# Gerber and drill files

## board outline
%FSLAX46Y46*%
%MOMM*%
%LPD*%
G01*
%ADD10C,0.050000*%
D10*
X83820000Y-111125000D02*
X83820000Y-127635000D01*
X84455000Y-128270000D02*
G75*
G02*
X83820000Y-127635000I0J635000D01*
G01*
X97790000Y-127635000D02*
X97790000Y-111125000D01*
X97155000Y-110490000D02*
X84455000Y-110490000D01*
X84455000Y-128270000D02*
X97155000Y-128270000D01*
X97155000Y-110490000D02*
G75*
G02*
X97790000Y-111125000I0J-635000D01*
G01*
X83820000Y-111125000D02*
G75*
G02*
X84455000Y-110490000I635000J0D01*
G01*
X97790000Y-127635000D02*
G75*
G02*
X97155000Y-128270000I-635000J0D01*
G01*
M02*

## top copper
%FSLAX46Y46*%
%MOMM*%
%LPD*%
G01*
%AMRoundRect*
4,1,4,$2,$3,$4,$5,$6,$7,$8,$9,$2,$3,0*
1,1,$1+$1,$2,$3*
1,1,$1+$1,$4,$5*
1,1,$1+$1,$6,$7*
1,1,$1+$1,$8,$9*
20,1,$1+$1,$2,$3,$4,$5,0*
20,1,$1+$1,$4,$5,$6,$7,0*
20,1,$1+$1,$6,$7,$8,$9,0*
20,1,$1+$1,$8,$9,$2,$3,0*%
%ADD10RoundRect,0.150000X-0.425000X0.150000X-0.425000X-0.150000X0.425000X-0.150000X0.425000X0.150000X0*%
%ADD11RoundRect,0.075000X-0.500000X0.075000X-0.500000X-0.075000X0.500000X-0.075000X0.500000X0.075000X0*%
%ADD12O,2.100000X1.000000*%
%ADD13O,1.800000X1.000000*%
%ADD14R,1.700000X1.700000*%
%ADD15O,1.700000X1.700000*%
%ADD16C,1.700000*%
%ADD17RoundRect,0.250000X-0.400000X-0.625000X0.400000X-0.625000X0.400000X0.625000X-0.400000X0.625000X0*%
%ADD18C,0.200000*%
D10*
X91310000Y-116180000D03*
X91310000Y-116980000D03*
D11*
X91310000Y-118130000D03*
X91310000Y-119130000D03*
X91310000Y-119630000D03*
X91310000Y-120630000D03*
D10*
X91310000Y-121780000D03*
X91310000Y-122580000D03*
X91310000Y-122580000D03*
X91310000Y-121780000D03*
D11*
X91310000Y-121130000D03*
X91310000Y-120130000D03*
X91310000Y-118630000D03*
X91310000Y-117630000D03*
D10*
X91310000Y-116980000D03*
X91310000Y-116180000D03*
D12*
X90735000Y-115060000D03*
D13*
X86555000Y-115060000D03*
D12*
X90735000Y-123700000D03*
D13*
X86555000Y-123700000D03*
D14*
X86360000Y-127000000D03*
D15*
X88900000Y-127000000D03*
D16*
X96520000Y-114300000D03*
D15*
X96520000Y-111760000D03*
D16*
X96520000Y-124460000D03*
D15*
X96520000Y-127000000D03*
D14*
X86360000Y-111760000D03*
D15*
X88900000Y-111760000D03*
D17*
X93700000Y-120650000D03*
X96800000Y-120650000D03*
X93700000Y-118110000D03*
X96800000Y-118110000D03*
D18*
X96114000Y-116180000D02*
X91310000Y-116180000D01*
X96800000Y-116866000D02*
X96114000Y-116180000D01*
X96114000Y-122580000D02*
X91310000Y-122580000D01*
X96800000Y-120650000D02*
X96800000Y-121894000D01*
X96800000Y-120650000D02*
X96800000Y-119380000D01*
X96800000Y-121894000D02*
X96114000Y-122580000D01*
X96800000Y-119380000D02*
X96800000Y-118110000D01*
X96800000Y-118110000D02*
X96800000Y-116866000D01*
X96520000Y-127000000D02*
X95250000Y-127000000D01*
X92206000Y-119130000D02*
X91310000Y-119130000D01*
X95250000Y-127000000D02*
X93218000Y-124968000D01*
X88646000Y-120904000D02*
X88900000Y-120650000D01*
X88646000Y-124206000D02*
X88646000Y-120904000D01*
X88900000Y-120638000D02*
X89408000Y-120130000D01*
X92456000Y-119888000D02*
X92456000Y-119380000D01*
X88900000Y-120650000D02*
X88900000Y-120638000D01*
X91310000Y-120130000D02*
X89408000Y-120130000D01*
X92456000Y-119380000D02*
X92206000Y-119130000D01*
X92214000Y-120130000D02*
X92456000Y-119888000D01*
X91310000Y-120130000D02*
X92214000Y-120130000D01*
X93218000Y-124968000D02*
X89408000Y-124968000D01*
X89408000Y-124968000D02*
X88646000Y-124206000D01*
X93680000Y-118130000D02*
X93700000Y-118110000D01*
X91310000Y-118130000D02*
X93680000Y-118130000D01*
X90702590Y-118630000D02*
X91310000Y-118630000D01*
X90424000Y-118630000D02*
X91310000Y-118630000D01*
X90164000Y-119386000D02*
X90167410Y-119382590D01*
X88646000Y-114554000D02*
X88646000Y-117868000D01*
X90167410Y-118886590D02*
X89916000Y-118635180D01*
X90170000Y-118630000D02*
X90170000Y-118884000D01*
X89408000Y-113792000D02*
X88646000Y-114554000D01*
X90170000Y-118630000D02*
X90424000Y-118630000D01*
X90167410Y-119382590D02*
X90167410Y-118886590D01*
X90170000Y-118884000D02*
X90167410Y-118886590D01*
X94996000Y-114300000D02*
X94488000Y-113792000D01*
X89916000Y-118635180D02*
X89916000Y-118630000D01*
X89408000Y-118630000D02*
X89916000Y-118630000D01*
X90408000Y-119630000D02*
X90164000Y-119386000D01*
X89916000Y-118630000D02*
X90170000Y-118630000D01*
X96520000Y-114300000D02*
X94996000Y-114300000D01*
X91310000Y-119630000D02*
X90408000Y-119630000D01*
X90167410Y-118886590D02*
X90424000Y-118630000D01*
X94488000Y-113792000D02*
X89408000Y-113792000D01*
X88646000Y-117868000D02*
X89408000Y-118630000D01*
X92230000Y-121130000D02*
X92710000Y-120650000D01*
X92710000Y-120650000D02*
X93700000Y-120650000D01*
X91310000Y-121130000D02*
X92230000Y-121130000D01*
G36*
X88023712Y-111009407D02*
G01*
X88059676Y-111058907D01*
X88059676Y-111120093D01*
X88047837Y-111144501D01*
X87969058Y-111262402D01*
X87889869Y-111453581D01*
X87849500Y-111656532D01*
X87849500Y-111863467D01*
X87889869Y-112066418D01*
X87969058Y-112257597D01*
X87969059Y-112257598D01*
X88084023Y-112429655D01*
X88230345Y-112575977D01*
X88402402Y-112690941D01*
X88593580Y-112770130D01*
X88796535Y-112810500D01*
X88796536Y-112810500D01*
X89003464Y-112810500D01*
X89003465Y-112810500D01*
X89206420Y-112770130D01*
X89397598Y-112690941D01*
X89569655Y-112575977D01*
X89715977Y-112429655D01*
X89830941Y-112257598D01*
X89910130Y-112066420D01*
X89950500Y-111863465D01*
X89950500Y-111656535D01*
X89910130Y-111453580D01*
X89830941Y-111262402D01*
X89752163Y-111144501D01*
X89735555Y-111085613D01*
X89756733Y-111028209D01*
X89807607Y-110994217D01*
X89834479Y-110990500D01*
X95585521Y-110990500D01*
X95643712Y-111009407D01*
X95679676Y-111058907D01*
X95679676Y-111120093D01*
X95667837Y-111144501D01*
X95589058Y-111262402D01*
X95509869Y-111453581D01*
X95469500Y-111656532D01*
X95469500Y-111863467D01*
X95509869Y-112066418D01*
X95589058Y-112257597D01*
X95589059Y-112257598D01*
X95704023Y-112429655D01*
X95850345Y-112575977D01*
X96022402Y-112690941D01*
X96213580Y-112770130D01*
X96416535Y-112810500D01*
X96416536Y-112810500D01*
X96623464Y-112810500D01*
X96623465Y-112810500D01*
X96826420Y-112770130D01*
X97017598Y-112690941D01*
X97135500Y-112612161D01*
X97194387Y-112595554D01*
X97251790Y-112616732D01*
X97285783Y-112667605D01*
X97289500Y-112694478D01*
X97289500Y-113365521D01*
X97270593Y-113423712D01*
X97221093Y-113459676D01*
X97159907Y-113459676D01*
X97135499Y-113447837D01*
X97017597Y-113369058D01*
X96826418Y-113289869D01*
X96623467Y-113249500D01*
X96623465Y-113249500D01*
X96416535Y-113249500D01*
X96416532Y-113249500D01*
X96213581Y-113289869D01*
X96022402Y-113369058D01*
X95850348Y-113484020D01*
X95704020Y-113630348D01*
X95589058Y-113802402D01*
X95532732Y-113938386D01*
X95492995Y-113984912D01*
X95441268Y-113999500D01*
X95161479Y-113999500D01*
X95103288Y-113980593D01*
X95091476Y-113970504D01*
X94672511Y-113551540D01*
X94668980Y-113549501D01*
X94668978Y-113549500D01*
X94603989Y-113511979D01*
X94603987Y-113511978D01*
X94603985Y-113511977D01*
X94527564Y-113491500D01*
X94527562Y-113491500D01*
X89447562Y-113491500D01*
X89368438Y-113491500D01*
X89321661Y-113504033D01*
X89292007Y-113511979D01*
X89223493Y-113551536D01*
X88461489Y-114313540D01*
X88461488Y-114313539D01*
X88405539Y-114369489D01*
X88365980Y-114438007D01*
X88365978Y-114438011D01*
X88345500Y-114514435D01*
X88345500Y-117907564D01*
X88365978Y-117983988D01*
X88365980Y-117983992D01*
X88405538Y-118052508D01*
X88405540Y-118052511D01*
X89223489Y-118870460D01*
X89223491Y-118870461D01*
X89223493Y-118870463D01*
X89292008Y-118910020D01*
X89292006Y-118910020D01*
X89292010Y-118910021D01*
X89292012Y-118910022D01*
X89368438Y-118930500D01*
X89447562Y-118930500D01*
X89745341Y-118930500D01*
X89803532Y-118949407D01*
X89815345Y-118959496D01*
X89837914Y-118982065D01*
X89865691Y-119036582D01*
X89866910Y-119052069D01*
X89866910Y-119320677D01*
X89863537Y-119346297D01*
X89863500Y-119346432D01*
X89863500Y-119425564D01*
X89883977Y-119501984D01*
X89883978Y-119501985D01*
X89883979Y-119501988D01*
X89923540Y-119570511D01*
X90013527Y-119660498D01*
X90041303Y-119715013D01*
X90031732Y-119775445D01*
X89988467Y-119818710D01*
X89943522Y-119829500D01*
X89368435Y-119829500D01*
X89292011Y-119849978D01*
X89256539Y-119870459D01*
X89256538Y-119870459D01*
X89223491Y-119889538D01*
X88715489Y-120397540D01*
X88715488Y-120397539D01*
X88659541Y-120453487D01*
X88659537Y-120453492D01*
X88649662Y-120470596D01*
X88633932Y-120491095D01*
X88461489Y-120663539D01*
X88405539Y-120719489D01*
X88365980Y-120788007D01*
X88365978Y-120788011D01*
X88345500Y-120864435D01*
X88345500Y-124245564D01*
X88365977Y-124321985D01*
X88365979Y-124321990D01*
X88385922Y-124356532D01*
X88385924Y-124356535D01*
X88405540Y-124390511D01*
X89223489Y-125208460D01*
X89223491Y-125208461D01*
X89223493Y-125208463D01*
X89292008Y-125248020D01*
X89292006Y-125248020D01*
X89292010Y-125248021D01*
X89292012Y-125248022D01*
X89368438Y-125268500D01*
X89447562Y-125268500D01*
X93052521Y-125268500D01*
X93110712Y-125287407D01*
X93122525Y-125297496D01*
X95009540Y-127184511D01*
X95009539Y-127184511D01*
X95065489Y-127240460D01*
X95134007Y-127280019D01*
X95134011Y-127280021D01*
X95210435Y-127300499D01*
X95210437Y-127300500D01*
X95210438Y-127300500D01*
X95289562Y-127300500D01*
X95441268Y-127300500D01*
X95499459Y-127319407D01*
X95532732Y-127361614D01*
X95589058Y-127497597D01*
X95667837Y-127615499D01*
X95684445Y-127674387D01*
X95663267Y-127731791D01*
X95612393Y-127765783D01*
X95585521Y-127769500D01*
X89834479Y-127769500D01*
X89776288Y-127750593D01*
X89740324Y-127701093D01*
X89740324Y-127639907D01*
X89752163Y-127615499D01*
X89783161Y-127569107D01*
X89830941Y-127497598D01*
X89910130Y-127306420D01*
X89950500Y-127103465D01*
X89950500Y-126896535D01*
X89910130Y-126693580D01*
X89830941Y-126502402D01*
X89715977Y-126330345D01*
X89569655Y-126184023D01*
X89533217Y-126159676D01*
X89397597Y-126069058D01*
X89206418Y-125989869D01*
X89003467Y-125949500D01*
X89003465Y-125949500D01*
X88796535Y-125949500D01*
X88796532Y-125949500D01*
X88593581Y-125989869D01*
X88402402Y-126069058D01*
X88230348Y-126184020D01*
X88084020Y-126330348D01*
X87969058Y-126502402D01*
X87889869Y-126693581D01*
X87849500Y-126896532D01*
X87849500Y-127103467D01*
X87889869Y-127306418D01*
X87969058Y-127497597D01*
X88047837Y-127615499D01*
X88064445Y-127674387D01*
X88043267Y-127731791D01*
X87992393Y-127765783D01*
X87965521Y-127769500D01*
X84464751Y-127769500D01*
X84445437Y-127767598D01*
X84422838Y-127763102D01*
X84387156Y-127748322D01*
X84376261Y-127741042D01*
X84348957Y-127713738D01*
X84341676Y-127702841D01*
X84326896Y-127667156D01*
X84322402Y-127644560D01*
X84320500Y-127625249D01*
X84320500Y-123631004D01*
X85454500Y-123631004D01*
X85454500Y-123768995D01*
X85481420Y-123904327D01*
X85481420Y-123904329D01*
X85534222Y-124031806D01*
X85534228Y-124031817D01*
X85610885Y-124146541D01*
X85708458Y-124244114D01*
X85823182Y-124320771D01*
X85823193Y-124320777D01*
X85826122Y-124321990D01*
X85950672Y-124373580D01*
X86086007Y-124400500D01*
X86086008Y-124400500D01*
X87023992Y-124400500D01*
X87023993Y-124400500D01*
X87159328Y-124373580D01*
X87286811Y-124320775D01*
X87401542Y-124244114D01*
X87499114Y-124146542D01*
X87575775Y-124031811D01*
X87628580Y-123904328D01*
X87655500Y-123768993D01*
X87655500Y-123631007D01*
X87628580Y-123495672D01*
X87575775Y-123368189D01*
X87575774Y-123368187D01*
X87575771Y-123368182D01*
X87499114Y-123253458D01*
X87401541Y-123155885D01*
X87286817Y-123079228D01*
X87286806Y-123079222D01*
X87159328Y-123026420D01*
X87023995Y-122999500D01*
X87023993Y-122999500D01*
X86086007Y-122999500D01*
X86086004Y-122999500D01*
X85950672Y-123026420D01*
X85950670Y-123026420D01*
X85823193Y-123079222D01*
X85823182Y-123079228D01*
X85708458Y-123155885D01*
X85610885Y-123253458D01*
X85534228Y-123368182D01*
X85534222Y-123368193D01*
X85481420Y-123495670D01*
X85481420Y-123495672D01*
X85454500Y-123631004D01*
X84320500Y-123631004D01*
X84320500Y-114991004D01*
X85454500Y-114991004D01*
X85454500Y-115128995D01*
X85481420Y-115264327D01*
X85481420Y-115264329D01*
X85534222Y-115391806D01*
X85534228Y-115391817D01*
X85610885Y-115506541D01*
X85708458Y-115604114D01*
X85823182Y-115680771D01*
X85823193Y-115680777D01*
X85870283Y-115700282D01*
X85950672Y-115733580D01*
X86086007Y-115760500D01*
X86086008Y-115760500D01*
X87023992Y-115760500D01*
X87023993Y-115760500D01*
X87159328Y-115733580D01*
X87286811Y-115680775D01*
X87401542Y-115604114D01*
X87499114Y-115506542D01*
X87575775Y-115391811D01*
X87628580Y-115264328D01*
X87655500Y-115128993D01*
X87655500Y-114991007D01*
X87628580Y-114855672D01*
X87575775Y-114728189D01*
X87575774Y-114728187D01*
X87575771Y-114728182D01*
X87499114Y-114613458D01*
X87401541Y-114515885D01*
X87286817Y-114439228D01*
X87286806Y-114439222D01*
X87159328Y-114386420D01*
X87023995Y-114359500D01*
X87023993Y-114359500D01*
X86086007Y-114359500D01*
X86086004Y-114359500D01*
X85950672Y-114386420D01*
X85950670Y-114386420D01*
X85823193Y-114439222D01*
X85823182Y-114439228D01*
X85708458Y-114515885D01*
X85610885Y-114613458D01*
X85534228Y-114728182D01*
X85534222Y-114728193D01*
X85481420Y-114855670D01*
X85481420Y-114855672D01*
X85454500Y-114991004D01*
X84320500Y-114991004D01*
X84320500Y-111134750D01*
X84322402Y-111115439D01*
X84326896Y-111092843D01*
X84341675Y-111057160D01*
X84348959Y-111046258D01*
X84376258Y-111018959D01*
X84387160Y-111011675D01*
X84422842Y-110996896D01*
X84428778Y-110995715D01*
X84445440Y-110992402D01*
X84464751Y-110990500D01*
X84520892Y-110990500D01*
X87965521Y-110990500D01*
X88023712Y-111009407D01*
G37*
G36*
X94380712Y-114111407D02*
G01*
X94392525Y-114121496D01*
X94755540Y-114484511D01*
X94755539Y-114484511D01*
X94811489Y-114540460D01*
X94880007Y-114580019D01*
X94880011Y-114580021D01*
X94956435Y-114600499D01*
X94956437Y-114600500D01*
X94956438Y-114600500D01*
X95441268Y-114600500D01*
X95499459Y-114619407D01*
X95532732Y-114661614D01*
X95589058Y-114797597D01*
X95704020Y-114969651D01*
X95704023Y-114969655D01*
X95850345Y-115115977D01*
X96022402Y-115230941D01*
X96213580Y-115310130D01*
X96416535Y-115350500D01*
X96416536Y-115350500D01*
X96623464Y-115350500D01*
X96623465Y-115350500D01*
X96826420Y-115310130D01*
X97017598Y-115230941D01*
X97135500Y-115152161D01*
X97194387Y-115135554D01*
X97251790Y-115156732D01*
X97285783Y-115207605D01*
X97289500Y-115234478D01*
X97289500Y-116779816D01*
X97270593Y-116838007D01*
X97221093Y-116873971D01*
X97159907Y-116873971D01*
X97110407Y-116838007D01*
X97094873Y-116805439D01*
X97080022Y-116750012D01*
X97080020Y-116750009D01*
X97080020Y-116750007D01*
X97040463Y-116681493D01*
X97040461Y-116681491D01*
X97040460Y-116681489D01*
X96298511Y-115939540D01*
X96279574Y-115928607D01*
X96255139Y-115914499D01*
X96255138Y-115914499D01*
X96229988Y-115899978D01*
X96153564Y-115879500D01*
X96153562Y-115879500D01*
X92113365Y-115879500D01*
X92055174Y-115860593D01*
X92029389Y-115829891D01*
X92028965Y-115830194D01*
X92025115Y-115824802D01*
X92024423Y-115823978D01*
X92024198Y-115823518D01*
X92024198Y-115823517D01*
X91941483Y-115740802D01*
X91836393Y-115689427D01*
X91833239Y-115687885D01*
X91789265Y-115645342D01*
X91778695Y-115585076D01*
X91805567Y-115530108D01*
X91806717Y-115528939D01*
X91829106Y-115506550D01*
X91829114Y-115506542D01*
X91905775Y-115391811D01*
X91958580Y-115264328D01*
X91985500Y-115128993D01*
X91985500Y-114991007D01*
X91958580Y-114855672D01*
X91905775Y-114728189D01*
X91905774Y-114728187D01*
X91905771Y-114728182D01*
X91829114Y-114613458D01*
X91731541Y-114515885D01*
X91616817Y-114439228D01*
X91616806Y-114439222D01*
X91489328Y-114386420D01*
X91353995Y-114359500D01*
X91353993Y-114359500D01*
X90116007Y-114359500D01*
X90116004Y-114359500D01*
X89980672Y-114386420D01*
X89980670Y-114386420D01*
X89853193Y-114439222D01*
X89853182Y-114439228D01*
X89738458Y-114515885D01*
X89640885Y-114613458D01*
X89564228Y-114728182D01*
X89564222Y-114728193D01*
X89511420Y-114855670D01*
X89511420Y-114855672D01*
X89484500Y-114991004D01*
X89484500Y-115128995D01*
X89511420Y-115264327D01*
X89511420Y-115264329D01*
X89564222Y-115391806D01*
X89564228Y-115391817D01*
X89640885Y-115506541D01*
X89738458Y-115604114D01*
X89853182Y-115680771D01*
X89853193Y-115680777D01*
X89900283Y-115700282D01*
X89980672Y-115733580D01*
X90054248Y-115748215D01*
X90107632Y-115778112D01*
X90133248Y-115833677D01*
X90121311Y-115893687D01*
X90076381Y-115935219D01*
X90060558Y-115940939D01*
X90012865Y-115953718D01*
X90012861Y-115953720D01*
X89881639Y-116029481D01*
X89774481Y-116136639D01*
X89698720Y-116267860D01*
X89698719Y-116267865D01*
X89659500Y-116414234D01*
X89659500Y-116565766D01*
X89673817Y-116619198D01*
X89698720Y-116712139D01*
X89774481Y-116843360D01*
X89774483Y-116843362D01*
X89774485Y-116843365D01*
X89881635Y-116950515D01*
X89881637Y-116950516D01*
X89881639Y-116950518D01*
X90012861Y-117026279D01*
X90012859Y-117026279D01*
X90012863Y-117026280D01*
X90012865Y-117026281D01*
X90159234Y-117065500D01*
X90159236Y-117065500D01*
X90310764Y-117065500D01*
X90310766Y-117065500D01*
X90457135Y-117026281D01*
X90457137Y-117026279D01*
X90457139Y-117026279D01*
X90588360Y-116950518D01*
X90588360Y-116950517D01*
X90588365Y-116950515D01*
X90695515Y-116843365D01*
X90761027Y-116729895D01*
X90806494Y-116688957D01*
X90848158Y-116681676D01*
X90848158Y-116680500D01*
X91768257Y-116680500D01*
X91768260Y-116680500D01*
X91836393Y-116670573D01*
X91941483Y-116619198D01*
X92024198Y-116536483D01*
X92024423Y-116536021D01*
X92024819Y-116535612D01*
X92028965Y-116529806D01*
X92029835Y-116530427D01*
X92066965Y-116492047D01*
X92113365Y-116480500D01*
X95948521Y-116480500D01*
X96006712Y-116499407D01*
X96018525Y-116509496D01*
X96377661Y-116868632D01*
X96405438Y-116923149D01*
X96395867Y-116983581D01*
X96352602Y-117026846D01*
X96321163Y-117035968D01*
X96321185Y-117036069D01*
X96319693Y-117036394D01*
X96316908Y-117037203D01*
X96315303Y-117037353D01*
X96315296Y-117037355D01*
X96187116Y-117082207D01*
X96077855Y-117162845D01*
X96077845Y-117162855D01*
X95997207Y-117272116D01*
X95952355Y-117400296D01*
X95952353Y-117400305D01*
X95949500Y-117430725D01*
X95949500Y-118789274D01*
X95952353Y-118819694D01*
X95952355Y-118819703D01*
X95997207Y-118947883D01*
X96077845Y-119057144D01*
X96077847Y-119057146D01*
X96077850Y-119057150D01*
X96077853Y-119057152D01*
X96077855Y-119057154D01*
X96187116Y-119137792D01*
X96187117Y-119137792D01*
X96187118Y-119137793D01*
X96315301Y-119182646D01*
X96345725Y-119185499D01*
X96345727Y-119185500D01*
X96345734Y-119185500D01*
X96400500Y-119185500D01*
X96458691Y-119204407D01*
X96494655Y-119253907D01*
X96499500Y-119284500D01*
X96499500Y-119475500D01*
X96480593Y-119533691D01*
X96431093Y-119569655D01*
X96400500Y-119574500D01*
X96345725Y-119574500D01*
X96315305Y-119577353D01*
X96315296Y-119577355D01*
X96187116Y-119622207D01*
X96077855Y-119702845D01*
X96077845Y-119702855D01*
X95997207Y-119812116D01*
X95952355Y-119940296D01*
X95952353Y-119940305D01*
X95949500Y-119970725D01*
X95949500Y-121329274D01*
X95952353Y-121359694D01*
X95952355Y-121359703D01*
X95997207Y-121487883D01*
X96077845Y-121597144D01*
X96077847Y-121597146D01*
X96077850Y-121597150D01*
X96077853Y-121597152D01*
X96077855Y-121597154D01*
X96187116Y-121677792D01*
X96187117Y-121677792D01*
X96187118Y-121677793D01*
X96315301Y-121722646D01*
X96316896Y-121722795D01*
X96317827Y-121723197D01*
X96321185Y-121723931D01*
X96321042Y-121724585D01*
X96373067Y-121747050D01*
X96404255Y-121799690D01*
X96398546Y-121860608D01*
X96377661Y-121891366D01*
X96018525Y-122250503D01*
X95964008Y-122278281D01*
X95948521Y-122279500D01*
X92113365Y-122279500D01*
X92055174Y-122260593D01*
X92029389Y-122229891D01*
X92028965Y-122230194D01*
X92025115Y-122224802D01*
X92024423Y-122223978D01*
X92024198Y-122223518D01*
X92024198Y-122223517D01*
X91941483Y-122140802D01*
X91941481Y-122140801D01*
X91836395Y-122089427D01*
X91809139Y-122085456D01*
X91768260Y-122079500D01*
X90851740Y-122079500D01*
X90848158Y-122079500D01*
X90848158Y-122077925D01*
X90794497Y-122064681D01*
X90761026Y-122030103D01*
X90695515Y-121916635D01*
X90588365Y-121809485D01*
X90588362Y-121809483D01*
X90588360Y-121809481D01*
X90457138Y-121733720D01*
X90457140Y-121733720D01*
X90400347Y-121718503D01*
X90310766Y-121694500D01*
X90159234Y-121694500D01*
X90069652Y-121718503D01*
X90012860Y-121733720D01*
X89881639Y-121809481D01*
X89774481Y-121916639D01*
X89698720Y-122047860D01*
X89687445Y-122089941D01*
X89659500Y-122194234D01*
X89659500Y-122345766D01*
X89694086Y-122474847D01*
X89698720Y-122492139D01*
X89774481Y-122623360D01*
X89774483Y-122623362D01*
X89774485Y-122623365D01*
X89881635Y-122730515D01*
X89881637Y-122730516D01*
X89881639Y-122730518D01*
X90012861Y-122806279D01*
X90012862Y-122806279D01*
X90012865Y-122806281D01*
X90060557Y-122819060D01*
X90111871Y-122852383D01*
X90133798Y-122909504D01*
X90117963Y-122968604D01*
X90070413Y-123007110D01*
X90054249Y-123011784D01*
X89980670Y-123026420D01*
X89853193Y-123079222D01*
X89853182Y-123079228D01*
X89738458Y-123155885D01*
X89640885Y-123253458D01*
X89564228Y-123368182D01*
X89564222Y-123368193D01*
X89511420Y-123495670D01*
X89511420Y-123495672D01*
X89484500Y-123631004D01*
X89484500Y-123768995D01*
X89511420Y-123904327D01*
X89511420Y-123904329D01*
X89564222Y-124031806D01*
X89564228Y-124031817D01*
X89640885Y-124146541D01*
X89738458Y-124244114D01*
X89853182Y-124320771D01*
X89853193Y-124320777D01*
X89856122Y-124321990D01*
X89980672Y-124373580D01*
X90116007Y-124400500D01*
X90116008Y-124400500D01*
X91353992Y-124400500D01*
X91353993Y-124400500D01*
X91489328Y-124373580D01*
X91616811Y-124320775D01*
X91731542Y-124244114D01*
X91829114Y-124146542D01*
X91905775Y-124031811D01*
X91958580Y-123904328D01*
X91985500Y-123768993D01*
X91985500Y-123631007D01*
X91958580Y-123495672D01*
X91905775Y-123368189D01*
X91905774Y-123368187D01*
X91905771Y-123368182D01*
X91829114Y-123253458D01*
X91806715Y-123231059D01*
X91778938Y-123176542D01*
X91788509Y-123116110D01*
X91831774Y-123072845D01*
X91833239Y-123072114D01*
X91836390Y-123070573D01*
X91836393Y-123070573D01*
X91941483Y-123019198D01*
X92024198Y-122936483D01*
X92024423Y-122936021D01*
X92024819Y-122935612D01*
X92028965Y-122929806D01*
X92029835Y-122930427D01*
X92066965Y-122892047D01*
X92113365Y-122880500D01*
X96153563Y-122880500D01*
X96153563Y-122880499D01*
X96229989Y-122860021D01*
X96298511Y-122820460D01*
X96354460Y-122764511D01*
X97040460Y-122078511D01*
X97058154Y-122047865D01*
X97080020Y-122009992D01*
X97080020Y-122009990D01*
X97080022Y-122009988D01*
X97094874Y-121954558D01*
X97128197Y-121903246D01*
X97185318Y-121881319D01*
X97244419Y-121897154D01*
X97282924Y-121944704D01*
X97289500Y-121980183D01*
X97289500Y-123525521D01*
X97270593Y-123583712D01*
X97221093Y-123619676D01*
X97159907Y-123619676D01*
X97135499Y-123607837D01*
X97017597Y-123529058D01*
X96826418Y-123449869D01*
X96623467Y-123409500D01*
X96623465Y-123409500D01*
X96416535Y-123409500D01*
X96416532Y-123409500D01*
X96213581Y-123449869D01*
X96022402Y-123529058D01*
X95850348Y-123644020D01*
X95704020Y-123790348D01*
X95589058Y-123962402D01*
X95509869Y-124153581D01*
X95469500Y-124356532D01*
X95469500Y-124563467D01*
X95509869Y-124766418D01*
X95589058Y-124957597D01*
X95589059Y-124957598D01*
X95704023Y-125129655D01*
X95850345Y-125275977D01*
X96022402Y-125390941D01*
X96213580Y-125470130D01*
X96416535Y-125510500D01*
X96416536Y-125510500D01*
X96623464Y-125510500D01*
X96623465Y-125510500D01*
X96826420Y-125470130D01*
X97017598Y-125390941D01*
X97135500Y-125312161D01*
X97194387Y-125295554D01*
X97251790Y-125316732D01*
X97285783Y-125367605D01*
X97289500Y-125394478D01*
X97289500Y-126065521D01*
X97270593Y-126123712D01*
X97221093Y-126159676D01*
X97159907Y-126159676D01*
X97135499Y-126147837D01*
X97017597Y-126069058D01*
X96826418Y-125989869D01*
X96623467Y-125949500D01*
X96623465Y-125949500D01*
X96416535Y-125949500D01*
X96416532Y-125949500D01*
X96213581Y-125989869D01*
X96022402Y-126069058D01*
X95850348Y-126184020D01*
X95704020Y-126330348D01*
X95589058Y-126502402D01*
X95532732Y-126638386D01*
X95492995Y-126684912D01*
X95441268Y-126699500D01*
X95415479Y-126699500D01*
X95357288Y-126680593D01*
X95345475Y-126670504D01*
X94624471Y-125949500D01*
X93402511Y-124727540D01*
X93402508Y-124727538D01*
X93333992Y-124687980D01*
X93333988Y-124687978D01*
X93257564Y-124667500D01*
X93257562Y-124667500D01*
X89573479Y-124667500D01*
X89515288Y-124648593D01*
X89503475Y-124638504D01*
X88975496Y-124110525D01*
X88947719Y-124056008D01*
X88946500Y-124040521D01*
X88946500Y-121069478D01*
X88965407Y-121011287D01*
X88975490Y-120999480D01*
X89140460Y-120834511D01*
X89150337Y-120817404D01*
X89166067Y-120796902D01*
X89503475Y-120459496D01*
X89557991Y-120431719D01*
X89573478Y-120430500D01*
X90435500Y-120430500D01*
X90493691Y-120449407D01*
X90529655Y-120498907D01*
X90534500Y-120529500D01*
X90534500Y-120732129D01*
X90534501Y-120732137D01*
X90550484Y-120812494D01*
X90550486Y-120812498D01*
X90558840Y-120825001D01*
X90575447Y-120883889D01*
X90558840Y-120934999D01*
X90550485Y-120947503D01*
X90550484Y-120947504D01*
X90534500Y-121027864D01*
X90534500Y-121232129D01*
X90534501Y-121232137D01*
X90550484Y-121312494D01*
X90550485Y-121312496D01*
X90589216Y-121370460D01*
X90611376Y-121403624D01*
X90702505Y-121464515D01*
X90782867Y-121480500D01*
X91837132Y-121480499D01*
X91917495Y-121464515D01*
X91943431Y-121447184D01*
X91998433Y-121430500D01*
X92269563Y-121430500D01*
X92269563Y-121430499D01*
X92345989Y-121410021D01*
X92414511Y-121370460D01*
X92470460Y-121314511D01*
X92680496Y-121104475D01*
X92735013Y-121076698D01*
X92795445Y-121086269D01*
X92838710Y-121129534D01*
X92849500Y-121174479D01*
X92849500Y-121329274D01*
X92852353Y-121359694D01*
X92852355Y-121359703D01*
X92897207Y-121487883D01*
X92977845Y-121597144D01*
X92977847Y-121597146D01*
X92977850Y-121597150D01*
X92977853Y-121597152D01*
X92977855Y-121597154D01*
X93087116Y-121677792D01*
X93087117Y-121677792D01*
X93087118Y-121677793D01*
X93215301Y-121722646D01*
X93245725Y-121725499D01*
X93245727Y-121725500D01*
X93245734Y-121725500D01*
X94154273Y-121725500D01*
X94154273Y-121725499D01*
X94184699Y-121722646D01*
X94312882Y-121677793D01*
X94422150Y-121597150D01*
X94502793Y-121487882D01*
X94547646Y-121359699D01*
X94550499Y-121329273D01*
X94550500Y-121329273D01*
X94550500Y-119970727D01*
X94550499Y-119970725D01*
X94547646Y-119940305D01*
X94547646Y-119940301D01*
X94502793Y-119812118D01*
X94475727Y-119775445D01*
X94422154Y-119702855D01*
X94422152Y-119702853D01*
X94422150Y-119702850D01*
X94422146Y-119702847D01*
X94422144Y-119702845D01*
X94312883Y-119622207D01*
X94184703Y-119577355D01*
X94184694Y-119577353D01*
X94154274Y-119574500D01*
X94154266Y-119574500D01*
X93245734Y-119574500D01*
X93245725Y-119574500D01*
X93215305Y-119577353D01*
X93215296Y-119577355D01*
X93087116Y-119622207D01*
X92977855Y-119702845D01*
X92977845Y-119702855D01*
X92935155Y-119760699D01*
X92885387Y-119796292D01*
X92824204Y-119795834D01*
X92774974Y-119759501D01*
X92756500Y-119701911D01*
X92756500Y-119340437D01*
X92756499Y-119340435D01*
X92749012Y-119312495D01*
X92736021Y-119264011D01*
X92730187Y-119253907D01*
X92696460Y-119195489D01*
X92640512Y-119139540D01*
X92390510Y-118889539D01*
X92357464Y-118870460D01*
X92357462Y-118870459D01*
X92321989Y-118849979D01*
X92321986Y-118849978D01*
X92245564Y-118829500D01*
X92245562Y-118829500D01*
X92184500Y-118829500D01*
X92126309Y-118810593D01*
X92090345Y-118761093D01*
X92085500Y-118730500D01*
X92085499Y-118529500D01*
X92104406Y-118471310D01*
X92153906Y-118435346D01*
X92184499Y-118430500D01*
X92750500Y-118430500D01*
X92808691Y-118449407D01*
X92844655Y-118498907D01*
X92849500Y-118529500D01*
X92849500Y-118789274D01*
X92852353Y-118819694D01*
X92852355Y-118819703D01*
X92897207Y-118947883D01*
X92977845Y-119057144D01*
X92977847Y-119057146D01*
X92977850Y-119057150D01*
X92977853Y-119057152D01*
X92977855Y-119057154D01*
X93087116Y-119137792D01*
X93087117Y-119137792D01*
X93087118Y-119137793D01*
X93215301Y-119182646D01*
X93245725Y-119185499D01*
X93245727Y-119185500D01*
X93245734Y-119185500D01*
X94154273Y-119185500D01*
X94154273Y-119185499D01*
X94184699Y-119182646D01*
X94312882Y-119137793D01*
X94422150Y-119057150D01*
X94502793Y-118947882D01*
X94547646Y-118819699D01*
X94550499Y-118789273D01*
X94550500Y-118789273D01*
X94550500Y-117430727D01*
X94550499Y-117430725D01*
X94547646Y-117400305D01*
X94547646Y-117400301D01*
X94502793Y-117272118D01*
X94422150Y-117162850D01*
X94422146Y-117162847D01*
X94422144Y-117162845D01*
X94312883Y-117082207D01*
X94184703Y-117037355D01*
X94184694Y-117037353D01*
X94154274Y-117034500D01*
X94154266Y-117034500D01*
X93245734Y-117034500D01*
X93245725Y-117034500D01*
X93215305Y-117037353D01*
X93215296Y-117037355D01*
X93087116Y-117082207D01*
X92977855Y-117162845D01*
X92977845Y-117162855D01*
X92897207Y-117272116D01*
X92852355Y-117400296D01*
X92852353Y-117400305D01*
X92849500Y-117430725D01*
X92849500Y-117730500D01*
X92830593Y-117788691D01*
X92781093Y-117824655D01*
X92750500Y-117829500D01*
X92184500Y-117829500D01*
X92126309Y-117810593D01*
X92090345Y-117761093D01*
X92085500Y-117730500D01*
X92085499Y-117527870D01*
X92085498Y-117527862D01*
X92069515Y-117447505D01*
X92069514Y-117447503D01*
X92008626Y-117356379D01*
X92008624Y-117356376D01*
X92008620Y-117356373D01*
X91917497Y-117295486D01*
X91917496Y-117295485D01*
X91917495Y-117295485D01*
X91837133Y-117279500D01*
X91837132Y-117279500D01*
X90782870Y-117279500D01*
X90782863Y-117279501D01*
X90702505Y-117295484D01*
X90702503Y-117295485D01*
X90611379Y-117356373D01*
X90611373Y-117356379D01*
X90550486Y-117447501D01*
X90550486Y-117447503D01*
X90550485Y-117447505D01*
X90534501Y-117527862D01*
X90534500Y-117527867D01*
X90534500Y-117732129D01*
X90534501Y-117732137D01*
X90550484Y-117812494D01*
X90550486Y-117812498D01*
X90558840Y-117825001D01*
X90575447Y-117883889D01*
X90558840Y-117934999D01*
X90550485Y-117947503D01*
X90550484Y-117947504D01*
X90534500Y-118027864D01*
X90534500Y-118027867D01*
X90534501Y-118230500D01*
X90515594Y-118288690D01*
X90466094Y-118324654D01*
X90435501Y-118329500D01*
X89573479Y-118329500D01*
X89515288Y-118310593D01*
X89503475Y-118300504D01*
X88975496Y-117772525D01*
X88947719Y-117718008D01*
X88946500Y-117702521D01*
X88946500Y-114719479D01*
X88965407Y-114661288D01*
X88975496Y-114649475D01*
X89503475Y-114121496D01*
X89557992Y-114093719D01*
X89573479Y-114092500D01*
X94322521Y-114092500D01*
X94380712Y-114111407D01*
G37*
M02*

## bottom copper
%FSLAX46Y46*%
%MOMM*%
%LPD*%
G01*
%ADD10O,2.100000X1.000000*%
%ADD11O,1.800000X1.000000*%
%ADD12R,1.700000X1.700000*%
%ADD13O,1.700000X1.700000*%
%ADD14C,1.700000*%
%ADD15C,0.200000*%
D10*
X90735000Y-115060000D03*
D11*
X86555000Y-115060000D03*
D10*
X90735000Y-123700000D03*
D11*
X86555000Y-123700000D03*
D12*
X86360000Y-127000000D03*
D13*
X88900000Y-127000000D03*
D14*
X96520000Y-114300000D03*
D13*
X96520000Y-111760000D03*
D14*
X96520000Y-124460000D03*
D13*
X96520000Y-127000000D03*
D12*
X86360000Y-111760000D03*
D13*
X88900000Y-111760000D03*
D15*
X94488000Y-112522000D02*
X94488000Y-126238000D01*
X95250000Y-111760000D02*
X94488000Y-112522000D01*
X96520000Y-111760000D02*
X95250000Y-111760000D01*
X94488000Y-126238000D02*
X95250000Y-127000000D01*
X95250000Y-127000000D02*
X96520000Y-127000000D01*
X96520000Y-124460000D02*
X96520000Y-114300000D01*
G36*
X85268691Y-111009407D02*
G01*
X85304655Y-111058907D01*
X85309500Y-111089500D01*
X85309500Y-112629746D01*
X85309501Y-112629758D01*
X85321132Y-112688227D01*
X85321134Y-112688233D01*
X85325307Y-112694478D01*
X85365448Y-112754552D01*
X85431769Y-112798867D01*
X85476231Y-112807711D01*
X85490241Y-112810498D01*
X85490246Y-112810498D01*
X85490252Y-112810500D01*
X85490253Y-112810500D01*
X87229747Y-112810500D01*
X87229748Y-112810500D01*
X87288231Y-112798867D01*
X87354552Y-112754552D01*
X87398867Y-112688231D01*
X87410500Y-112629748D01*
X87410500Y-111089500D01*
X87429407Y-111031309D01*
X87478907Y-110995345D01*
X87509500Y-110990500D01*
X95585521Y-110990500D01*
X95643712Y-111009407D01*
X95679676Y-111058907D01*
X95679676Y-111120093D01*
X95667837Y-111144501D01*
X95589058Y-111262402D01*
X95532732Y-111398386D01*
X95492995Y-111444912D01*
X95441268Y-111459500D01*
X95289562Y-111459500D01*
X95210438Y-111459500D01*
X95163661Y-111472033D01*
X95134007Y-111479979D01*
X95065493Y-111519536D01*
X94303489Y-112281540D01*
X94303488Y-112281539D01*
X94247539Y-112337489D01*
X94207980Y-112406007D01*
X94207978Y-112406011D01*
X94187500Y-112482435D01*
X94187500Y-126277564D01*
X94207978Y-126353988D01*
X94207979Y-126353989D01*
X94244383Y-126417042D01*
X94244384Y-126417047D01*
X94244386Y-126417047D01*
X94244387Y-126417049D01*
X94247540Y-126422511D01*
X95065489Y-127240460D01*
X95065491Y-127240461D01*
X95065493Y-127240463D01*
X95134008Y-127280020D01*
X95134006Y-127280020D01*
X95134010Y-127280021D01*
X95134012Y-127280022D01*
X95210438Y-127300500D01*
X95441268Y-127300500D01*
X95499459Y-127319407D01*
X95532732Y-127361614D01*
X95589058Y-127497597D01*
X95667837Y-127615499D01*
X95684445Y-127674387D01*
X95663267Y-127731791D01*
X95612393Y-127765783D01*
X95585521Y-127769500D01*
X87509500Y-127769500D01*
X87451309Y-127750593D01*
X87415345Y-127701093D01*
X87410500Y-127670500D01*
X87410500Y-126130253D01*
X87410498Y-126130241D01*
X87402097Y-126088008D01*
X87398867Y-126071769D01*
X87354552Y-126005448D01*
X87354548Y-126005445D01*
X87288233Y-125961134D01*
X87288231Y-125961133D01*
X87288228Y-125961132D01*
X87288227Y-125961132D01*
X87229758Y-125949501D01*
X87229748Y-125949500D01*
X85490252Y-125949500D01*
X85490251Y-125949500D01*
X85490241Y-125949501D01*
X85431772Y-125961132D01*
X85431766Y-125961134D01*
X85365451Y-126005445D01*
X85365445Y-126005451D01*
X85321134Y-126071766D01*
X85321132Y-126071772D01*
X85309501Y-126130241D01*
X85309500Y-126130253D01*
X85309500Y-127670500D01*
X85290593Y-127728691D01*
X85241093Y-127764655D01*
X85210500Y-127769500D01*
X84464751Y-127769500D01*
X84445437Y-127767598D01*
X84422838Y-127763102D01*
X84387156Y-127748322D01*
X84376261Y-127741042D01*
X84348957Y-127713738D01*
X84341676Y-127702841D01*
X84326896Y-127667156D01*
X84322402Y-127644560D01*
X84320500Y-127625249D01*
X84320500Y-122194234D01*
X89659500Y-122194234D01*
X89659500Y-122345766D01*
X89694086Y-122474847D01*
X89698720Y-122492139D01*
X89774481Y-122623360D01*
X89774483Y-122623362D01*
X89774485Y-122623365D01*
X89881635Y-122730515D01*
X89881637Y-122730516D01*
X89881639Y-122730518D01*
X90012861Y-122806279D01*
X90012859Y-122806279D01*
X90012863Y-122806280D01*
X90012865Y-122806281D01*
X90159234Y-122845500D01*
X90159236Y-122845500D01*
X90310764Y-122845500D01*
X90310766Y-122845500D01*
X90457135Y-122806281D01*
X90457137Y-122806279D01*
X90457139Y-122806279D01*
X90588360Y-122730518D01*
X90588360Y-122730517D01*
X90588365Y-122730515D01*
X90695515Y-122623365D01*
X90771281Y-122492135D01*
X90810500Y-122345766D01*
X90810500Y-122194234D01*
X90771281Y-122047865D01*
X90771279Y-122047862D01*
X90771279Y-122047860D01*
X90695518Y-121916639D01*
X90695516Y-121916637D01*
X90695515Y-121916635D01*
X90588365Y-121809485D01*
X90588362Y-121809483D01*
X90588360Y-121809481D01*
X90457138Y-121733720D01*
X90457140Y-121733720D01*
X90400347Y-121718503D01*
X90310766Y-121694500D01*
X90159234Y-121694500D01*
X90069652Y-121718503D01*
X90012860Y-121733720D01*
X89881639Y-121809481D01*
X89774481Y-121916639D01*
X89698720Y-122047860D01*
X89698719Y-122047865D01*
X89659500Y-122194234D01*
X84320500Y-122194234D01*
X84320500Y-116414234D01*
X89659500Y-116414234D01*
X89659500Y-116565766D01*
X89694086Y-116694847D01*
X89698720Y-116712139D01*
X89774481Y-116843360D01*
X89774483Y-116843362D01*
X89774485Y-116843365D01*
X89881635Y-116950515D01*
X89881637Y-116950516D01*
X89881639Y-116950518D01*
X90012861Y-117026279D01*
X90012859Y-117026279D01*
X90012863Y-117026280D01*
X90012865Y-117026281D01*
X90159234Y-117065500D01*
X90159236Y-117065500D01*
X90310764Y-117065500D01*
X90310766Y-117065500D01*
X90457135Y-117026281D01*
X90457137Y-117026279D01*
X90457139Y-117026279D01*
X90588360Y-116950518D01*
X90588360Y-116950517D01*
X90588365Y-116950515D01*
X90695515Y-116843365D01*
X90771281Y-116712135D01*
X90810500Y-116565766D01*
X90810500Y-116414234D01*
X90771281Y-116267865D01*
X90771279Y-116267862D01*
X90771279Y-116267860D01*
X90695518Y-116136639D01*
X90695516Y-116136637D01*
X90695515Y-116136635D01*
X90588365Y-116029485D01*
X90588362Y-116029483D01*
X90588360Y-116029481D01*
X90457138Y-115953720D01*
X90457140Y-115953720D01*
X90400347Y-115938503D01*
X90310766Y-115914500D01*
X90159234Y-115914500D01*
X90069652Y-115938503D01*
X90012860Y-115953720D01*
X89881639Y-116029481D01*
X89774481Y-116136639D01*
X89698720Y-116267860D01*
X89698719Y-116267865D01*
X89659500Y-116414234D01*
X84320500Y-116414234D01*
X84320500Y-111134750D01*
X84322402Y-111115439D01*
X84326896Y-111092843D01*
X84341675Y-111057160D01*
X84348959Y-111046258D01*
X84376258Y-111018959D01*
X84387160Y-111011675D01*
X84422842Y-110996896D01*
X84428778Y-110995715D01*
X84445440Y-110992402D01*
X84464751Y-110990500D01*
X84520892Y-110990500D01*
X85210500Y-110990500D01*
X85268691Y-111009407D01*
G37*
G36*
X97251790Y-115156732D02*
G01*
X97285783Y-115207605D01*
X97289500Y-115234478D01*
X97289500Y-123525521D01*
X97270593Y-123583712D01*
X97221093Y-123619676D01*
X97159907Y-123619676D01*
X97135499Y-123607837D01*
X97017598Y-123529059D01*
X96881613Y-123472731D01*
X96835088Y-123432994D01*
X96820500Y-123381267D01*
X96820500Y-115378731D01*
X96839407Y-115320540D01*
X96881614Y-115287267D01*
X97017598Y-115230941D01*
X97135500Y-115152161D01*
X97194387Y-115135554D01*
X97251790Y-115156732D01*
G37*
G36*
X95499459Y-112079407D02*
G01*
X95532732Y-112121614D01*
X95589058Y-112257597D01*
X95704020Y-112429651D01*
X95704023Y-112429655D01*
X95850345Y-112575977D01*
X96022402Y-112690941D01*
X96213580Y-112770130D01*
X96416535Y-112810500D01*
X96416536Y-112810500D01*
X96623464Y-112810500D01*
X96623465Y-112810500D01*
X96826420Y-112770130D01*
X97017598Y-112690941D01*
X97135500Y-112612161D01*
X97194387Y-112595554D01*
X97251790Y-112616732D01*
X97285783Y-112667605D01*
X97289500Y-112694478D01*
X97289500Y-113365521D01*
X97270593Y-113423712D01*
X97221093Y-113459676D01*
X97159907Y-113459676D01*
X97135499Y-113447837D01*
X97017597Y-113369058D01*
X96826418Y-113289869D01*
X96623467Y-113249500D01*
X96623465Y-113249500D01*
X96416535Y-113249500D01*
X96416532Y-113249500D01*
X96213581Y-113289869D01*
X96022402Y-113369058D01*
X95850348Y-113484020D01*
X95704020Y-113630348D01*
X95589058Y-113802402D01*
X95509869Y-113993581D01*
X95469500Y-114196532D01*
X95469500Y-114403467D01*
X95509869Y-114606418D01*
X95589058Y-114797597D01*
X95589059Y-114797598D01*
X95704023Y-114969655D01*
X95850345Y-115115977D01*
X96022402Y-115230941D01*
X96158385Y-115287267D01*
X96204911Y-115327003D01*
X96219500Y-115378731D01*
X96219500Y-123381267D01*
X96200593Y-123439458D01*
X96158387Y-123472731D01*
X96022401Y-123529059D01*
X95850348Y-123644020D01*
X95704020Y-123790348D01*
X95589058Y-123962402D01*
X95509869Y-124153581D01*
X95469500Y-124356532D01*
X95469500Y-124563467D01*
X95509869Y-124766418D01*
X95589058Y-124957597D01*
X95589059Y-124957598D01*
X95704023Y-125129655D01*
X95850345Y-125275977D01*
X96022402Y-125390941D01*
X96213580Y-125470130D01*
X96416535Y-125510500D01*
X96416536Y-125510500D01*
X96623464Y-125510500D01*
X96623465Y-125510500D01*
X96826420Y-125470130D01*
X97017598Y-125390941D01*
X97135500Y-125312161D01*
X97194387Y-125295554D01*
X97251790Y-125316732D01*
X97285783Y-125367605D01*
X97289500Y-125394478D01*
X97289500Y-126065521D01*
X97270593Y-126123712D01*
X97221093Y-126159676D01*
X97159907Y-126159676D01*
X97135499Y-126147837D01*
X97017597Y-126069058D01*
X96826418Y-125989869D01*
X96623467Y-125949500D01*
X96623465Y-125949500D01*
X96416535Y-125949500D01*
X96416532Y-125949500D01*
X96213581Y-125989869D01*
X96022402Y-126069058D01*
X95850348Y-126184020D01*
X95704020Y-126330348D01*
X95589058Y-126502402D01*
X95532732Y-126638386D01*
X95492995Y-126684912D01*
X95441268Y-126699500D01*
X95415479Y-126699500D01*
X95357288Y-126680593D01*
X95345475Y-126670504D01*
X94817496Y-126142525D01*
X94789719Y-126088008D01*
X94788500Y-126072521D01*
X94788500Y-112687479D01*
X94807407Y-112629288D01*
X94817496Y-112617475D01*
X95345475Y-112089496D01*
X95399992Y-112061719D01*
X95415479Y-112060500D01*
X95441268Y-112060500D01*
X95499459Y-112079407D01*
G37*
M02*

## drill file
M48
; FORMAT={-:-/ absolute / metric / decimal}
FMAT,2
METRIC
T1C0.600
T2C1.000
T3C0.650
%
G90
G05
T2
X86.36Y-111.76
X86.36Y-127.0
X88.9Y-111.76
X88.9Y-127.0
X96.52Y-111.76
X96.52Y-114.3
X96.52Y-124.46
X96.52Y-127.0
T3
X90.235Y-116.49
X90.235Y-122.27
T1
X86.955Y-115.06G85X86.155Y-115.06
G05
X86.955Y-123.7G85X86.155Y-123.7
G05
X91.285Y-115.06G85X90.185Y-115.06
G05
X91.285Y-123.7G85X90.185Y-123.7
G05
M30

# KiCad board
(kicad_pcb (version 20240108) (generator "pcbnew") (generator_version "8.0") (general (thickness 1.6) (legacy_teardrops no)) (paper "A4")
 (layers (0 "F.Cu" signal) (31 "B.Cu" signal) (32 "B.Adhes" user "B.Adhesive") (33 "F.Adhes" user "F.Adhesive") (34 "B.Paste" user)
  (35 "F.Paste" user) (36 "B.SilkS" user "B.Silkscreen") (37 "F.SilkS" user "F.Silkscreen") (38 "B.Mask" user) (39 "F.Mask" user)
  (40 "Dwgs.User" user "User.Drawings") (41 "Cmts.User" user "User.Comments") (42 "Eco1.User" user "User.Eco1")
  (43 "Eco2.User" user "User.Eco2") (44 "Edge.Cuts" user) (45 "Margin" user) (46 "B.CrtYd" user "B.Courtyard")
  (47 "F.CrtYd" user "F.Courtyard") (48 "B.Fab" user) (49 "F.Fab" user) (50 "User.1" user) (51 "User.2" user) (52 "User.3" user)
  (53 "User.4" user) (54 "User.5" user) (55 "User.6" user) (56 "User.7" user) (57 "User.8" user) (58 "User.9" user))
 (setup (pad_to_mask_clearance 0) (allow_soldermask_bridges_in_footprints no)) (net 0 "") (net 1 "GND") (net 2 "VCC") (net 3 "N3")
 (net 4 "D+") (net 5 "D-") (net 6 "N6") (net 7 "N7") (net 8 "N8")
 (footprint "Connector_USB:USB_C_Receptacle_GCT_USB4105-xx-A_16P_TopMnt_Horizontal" (layer "F.Cu") (at 87.63 119.38 -90)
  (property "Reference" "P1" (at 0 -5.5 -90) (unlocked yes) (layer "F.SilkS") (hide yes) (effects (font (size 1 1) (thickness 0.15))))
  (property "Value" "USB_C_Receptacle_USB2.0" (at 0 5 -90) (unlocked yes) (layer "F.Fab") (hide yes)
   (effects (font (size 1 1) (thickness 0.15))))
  (pad "" np_thru_hole circle (at -2.89 -2.605 270) (size 0.65 0.65) (drill 0.65) (layers "F&B.Cu" "*.Mask"))
  (pad "" np_thru_hole circle (at 2.89 -2.605 270) (size 0.65 0.65) (drill 0.65) (layers "F&B.Cu" "*.Mask"))
  (pad "A1" smd roundrect (at -3.2 -3.68 270) (size 0.6 1.15) (layers "F.Cu" "F.Paste" "F.Mask") (roundrect_rratio 0.25) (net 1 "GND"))
  (pad "A4" smd roundrect (at -2.4 -3.68 270) (size 0.6 1.15) (layers "F.Cu" "F.Paste" "F.Mask") (roundrect_rratio 0.25) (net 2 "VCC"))
  (pad "A5" smd roundrect (at -1.25 -3.68 270) (size 0.3 1.15) (layers "F.Cu" "F.Paste" "F.Mask") (roundrect_rratio 0.25) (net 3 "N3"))
  (pad "A6" smd roundrect (at -0.25 -3.68 270) (size 0.3 1.15) (layers "F.Cu" "F.Paste" "F.Mask") (roundrect_rratio 0.25) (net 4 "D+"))
  (pad "A7" smd roundrect (at 0.25 -3.68 270) (size 0.3 1.15) (layers "F.Cu" "F.Paste" "F.Mask") (roundrect_rratio 0.25) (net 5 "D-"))
  (pad "A8" smd roundrect (at 1.25 -3.68 270) (size 0.3 1.15) (layers "F.Cu" "F.Paste" "F.Mask") (roundrect_rratio 0.25) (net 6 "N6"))
  (pad "A9" smd roundrect (at 2.4 -3.68 270) (size 0.6 1.15) (layers "F.Cu" "F.Paste" "F.Mask") (roundrect_rratio 0.25) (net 2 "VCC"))
  (pad "A12" smd roundrect (at 3.2 -3.68 270) (size 0.6 1.15) (layers "F.Cu" "F.Paste" "F.Mask") (roundrect_rratio 0.25) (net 1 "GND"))
  (pad "B1" smd roundrect (at 3.2 -3.68 270) (size 0.6 1.15) (layers "F.Cu" "F.Paste" "F.Mask") (roundrect_rratio 0.25) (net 1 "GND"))
  (pad "B4" smd roundrect (at 2.4 -3.68 270) (size 0.6 1.15) (layers "F.Cu" "F.Paste" "F.Mask") (roundrect_rratio 0.25) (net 2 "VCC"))
  (pad "B5" smd roundrect (at 1.75 -3.68 270) (size 0.3 1.15) (layers "F.Cu" "F.Paste" "F.Mask") (roundrect_rratio 0.25) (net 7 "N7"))
  (pad "B6" smd roundrect (at 0.75 -3.68 270) (size 0.3 1.15) (layers "F.Cu" "F.Paste" "F.Mask") (roundrect_rratio 0.25) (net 4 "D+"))
  (pad "B7" smd roundrect (at -0.75 -3.68 270) (size 0.3 1.15) (layers "F.Cu" "F.Paste" "F.Mask") (roundrect_rratio 0.25) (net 5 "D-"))
  (pad "B8" smd roundrect (at -1.75 -3.68 270) (size 0.3 1.15) (layers "F.Cu" "F.Paste" "F.Mask") (roundrect_rratio 0.25) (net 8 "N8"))
  (pad "B9" smd roundrect (at -2.4 -3.68 270) (size 0.6 1.15) (layers "F.Cu" "F.Paste" "F.Mask") (roundrect_rratio 0.25) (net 2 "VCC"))
  (pad "B12" smd roundrect (at -3.2 -3.68 270) (size 0.6 1.15) (layers "F.Cu" "F.Paste" "F.Mask") (roundrect_rratio 0.25) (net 1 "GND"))
  (pad "S1" thru_hole oval (at -4.32 -3.105 270) (size 1 2.1) (drill oval 0.6 1.7) (layers "*.Cu" "*.Mask" "F.Paste")
   (remove_unused_layers no) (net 1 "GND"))
  (pad "S1" thru_hole oval (at -4.32 1.075 270) (size 1 1.8) (drill oval 0.6 1.4) (layers "*.Cu" "*.Mask" "F.Paste")
   (remove_unused_layers no) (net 1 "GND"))
  (pad "S1" thru_hole oval (at 4.32 -3.105 270) (size 1 2.1) (drill oval 0.6 1.7) (layers "*.Cu" "*.Mask" "F.Paste")
   (remove_unused_layers no) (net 1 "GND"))
  (pad "S1" thru_hole oval (at 4.32 1.075 270) (size 1 1.8) (drill oval 0.6 1.4) (layers "*.Cu" "*.Mask" "F.Paste")
   (remove_unused_layers no) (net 1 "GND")))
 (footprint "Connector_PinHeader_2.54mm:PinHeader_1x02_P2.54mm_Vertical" (layer "F.Cu") (at 86.36 127 90)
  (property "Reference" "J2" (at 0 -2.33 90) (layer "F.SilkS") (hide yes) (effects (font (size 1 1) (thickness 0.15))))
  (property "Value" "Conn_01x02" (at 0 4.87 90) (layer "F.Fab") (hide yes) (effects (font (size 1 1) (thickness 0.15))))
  (pad "1" thru_hole rect (at 0 0 90) (size 1.7 1.7) (drill 1) (layers "*.Cu" "*.Mask") (remove_unused_layers no) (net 2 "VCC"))
  (pad "2" thru_hole oval (at 0 2.54 90) (size 1.7 1.7) (drill 1) (layers "*.Cu" "*.Mask") (remove_unused_layers no) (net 1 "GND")))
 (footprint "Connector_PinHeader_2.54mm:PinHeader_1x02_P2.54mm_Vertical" (layer "F.Cu") (at 96.52 114.3 180)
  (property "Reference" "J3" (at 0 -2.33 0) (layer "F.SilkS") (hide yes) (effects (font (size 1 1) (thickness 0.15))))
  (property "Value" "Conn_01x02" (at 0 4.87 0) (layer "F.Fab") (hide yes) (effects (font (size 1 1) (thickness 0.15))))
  (pad "1" thru_hole circle (at 0 0 180) (size 1.7 1.7) (drill 1) (layers "*.Cu" "*.Mask") (remove_unused_layers no) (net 5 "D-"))
  (pad "2" thru_hole oval (at 0 2.54 180) (size 1.7 1.7) (drill 1) (layers "*.Cu" "*.Mask") (remove_unused_layers no) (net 4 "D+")))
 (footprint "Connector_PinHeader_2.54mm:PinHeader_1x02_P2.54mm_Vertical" (layer "F.Cu") (at 96.52 124.46)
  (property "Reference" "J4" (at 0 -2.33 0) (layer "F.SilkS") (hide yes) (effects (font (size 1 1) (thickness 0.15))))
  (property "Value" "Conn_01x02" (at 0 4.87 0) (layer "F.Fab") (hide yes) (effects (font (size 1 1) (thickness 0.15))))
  (pad "1" thru_hole circle (at 0 0) (size 1.7 1.7) (drill 1) (layers "*.Cu" "*.Mask") (remove_unused_layers no) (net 5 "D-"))
  (pad "2" thru_hole oval (at 0 2.54) (size 1.7 1.7) (drill 1) (layers "*.Cu" "*.Mask") (remove_unused_layers no) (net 4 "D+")))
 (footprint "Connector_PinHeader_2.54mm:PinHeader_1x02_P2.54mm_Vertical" (layer "F.Cu") (at 86.36 111.76 90)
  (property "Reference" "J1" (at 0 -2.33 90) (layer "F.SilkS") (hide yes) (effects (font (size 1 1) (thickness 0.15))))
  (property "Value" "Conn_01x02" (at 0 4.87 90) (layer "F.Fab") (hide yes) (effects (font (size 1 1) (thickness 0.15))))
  (pad "1" thru_hole rect (at 0 0 90) (size 1.7 1.7) (drill 1) (layers "*.Cu" "*.Mask") (remove_unused_layers no) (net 2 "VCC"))
  (pad "2" thru_hole oval (at 0 2.54 90) (size 1.7 1.7) (drill 1) (layers "*.Cu" "*.Mask") (remove_unused_layers no) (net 1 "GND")))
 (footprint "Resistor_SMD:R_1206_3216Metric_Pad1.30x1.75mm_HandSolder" (layer "F.Cu") (at 95.25 120.65)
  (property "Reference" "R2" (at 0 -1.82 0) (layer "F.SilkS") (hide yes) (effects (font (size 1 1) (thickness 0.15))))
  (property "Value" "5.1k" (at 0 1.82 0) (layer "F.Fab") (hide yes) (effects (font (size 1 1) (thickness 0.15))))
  (pad "1" smd roundrect (at -1.55 0) (size 1.3 1.75) (layers "F.Cu" "F.Paste" "F.Mask") (roundrect_rratio 0.192308) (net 7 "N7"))
  (pad "2" smd roundrect (at 1.55 0) (size 1.3 1.75) (layers "F.Cu" "F.Paste" "F.Mask") (roundrect_rratio 0.192308) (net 1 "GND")))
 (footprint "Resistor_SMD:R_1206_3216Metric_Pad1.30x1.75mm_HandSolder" (layer "F.Cu") (at 95.25 118.11)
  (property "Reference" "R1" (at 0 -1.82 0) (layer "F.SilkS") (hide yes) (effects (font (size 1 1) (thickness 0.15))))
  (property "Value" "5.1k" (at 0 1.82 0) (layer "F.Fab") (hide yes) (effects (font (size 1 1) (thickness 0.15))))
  (pad "1" smd roundrect (at -1.55 0) (size 1.3 1.75) (layers "F.Cu" "F.Paste" "F.Mask") (roundrect_rratio 0.192308) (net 3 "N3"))
  (pad "2" smd roundrect (at 1.55 0) (size 1.3 1.75) (layers "F.Cu" "F.Paste" "F.Mask") (roundrect_rratio 0.192308) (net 1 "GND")))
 (gr_line (start 83.82 111.125) (end 83.82 127.635) (stroke (width 0.05) (type default)) (layer "Edge.Cuts"))
 (gr_arc (start 84.455 128.27) (mid 84.005987 128.084013) (end 83.82 127.635) (stroke (width 0.05) (type default)) (layer "Edge.Cuts"))
 (gr_line (start 97.79 127.635) (end 97.79 111.125) (stroke (width 0.05) (type default)) (layer "Edge.Cuts"))
 (gr_line (start 97.155 110.49) (end 84.455 110.49) (stroke (width 0.05) (type default)) (layer "Edge.Cuts"))
 (gr_line (start 84.455 128.27) (end 97.155 128.27) (stroke (width 0.05) (type default)) (layer "Edge.Cuts"))
 (gr_arc (start 97.155 110.49) (mid 97.604013 110.675987) (end 97.79 111.125) (stroke (width 0.05) (type default)) (layer "Edge.Cuts"))
 (gr_arc (start 83.82 111.125) (mid 84.005987 110.675987) (end 84.455 110.49) (stroke (width 0.05) (type default)) (layer "Edge.Cuts"))
 (gr_arc (start 97.79 127.635) (mid 97.604013 128.084013) (end 97.155 128.27) (stroke (width 0.05) (type default)) (layer "Edge.Cuts"))
 (segment (start 96.114 116.18) (end 91.31 116.18) (width 0.2) (layer "F.Cu") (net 1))
 (segment (start 96.8 116.866) (end 96.114 116.18) (width 0.2) (layer "F.Cu") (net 1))
 (segment (start 96.114 122.58) (end 91.31 122.58) (width 0.2) (layer "F.Cu") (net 1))
 (segment (start 96.8 120.65) (end 96.8 121.894) (width 0.2) (layer "F.Cu") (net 1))
 (segment (start 96.8 120.65) (end 96.8 119.38) (width 0.2) (layer "F.Cu") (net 1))
 (segment (start 96.8 121.894) (end 96.114 122.58) (width 0.2) (layer "F.Cu") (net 1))
 (segment (start 96.8 119.38) (end 96.8 118.11) (width 0.2) (layer "F.Cu") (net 1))
 (segment (start 96.8 118.11) (end 96.8 116.866) (width 0.2) (layer "F.Cu") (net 1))
 (segment (start 96.52 127) (end 95.25 127) (width 0.2) (layer "F.Cu") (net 4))
 (segment (start 92.206 119.13) (end 91.31 119.13) (width 0.2) (layer "F.Cu") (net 4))
 (segment (start 95.25 127) (end 93.218 124.968) (width 0.2) (layer "F.Cu") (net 4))
 (segment (start 88.646 120.904) (end 88.9 120.65) (width 0.2) (layer "F.Cu") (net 4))
 (segment (start 88.646 124.206) (end 88.646 120.904) (width 0.2) (layer "F.Cu") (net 4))
 (segment (start 88.9 120.638) (end 89.408 120.13) (width 0.2) (layer "F.Cu") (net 4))
 (segment (start 92.456 119.888) (end 92.456 119.38) (width 0.2) (layer "F.Cu") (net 4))
 (segment (start 88.9 120.65) (end 88.9 120.638) (width 0.2) (layer "F.Cu") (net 4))
 (segment (start 91.31 120.13) (end 89.408 120.13) (width 0.2) (layer "F.Cu") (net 4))
 (segment (start 92.456 119.38) (end 92.206 119.13) (width 0.2) (layer "F.Cu") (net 4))
 (segment (start 92.214 120.13) (end 92.456 119.888) (width 0.2) (layer "F.Cu") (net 4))
 (segment (start 91.31 120.13) (end 92.214 120.13) (width 0.2) (layer "F.Cu") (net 4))
 (segment (start 93.218 124.968) (end 89.408 124.968) (width 0.2) (layer "F.Cu") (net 4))
 (segment (start 89.408 124.968) (end 88.646 124.206) (width 0.2) (layer "F.Cu") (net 4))
 (segment (start 94.488 112.522) (end 94.488 126.238) (width 0.2) (layer "B.Cu") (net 4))
 (segment (start 95.25 111.76) (end 94.488 112.522) (width 0.2) (layer "B.Cu") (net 4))
 (segment (start 96.52 111.76) (end 95.25 111.76) (width 0.2) (layer "B.Cu") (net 4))
 (segment (start 94.488 126.238) (end 95.25 127) (width 0.2) (layer "B.Cu") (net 4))
 (segment (start 95.25 127) (end 96.52 127) (width 0.2) (layer "B.Cu") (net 4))
 (segment (start 93.68 118.13) (end 93.7 118.11) (width 0.2) (layer "F.Cu") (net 3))
 (segment (start 91.31 118.13) (end 93.68 118.13) (width 0.2) (layer "F.Cu") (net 3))
 (segment (start 90.70259 118.63) (end 91.31 118.63) (width 0.2) (layer "F.Cu") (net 5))
 (segment (start 90.424 118.63) (end 91.31 118.63) (width 0.2) (layer "F.Cu") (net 5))
 (segment (start 90.164 119.386) (end 90.16741 119.38259) (width 0.2) (layer "F.Cu") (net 5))
 (segment (start 88.646 114.554) (end 88.646 117.868) (width 0.2) (layer "F.Cu") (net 5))
 (segment (start 90.16741 118.88659) (end 89.916 118.63518) (width 0.2) (layer "F.Cu") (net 5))
 (segment (start 90.17 118.63) (end 90.17 118.884) (width 0.2) (layer "F.Cu") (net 5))
 (segment (start 89.408 113.792) (end 88.646 114.554) (width 0.2) (layer "F.Cu") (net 5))
 (segment (start 90.17 118.63) (end 90.424 118.63) (width 0.2) (layer "F.Cu") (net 5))
 (segment (start 90.16741 119.38259) (end 90.16741 118.88659) (width 0.2) (layer "F.Cu") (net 5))
 (segment (start 90.17 118.884) (end 90.16741 118.88659) (width 0.2) (layer "F.Cu") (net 5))
 (segment (start 94.996 114.3) (end 94.488 113.792) (width 0.2) (layer "F.Cu") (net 5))
 (segment (start 89.916 118.63518) (end 89.916 118.63) (width 0.2) (layer "F.Cu") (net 5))
 (segment (start 89.408 118.63) (end 89.916 118.63) (width 0.2) (layer "F.Cu") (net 5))
 (segment (start 90.408 119.63) (end 90.164 119.386) (width 0.2) (layer "F.Cu") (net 5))
 (segment (start 89.916 118.63) (end 90.17 118.63) (width 0.2) (layer "F.Cu") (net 5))
 (segment (start 96.52 114.3) (end 94.996 114.3) (width 0.2) (layer "F.Cu") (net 5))
 (segment (start 91.31 119.63) (end 90.408 119.63) (width 0.2) (layer "F.Cu") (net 5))
 (segment (start 90.16741 118.88659) (end 90.424 118.63) (width 0.2) (layer "F.Cu") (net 5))
 (segment (start 94.488 113.792) (end 89.408 113.792) (width 0.2) (layer "F.Cu") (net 5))
 (segment (start 88.646 117.868) (end 89.408 118.63) (width 0.2) (layer "F.Cu") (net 5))
 (segment (start 96.52 124.46) (end 96.52 114.3) (width 0.2) (layer "B.Cu") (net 5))
 (segment (start 92.23 121.13) (end 92.71 120.65) (width 0.2) (layer "F.Cu") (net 7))
 (segment (start 92.71 120.65) (end 93.7 120.65) (width 0.2) (layer "F.Cu") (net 7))
 (segment (start 91.31 121.13) (end 92.23 121.13) (width 0.2) (layer "F.Cu") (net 7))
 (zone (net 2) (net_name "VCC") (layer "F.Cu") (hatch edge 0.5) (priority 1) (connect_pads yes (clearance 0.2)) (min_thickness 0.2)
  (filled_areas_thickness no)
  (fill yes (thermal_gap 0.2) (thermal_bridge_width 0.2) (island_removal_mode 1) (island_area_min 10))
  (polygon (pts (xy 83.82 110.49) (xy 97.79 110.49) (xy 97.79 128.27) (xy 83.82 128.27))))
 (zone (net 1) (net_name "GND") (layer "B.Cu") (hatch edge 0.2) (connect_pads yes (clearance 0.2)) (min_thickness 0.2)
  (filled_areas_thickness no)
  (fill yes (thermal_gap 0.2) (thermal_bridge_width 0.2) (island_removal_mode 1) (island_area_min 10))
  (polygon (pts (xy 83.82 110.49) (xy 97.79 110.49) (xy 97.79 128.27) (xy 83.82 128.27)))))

